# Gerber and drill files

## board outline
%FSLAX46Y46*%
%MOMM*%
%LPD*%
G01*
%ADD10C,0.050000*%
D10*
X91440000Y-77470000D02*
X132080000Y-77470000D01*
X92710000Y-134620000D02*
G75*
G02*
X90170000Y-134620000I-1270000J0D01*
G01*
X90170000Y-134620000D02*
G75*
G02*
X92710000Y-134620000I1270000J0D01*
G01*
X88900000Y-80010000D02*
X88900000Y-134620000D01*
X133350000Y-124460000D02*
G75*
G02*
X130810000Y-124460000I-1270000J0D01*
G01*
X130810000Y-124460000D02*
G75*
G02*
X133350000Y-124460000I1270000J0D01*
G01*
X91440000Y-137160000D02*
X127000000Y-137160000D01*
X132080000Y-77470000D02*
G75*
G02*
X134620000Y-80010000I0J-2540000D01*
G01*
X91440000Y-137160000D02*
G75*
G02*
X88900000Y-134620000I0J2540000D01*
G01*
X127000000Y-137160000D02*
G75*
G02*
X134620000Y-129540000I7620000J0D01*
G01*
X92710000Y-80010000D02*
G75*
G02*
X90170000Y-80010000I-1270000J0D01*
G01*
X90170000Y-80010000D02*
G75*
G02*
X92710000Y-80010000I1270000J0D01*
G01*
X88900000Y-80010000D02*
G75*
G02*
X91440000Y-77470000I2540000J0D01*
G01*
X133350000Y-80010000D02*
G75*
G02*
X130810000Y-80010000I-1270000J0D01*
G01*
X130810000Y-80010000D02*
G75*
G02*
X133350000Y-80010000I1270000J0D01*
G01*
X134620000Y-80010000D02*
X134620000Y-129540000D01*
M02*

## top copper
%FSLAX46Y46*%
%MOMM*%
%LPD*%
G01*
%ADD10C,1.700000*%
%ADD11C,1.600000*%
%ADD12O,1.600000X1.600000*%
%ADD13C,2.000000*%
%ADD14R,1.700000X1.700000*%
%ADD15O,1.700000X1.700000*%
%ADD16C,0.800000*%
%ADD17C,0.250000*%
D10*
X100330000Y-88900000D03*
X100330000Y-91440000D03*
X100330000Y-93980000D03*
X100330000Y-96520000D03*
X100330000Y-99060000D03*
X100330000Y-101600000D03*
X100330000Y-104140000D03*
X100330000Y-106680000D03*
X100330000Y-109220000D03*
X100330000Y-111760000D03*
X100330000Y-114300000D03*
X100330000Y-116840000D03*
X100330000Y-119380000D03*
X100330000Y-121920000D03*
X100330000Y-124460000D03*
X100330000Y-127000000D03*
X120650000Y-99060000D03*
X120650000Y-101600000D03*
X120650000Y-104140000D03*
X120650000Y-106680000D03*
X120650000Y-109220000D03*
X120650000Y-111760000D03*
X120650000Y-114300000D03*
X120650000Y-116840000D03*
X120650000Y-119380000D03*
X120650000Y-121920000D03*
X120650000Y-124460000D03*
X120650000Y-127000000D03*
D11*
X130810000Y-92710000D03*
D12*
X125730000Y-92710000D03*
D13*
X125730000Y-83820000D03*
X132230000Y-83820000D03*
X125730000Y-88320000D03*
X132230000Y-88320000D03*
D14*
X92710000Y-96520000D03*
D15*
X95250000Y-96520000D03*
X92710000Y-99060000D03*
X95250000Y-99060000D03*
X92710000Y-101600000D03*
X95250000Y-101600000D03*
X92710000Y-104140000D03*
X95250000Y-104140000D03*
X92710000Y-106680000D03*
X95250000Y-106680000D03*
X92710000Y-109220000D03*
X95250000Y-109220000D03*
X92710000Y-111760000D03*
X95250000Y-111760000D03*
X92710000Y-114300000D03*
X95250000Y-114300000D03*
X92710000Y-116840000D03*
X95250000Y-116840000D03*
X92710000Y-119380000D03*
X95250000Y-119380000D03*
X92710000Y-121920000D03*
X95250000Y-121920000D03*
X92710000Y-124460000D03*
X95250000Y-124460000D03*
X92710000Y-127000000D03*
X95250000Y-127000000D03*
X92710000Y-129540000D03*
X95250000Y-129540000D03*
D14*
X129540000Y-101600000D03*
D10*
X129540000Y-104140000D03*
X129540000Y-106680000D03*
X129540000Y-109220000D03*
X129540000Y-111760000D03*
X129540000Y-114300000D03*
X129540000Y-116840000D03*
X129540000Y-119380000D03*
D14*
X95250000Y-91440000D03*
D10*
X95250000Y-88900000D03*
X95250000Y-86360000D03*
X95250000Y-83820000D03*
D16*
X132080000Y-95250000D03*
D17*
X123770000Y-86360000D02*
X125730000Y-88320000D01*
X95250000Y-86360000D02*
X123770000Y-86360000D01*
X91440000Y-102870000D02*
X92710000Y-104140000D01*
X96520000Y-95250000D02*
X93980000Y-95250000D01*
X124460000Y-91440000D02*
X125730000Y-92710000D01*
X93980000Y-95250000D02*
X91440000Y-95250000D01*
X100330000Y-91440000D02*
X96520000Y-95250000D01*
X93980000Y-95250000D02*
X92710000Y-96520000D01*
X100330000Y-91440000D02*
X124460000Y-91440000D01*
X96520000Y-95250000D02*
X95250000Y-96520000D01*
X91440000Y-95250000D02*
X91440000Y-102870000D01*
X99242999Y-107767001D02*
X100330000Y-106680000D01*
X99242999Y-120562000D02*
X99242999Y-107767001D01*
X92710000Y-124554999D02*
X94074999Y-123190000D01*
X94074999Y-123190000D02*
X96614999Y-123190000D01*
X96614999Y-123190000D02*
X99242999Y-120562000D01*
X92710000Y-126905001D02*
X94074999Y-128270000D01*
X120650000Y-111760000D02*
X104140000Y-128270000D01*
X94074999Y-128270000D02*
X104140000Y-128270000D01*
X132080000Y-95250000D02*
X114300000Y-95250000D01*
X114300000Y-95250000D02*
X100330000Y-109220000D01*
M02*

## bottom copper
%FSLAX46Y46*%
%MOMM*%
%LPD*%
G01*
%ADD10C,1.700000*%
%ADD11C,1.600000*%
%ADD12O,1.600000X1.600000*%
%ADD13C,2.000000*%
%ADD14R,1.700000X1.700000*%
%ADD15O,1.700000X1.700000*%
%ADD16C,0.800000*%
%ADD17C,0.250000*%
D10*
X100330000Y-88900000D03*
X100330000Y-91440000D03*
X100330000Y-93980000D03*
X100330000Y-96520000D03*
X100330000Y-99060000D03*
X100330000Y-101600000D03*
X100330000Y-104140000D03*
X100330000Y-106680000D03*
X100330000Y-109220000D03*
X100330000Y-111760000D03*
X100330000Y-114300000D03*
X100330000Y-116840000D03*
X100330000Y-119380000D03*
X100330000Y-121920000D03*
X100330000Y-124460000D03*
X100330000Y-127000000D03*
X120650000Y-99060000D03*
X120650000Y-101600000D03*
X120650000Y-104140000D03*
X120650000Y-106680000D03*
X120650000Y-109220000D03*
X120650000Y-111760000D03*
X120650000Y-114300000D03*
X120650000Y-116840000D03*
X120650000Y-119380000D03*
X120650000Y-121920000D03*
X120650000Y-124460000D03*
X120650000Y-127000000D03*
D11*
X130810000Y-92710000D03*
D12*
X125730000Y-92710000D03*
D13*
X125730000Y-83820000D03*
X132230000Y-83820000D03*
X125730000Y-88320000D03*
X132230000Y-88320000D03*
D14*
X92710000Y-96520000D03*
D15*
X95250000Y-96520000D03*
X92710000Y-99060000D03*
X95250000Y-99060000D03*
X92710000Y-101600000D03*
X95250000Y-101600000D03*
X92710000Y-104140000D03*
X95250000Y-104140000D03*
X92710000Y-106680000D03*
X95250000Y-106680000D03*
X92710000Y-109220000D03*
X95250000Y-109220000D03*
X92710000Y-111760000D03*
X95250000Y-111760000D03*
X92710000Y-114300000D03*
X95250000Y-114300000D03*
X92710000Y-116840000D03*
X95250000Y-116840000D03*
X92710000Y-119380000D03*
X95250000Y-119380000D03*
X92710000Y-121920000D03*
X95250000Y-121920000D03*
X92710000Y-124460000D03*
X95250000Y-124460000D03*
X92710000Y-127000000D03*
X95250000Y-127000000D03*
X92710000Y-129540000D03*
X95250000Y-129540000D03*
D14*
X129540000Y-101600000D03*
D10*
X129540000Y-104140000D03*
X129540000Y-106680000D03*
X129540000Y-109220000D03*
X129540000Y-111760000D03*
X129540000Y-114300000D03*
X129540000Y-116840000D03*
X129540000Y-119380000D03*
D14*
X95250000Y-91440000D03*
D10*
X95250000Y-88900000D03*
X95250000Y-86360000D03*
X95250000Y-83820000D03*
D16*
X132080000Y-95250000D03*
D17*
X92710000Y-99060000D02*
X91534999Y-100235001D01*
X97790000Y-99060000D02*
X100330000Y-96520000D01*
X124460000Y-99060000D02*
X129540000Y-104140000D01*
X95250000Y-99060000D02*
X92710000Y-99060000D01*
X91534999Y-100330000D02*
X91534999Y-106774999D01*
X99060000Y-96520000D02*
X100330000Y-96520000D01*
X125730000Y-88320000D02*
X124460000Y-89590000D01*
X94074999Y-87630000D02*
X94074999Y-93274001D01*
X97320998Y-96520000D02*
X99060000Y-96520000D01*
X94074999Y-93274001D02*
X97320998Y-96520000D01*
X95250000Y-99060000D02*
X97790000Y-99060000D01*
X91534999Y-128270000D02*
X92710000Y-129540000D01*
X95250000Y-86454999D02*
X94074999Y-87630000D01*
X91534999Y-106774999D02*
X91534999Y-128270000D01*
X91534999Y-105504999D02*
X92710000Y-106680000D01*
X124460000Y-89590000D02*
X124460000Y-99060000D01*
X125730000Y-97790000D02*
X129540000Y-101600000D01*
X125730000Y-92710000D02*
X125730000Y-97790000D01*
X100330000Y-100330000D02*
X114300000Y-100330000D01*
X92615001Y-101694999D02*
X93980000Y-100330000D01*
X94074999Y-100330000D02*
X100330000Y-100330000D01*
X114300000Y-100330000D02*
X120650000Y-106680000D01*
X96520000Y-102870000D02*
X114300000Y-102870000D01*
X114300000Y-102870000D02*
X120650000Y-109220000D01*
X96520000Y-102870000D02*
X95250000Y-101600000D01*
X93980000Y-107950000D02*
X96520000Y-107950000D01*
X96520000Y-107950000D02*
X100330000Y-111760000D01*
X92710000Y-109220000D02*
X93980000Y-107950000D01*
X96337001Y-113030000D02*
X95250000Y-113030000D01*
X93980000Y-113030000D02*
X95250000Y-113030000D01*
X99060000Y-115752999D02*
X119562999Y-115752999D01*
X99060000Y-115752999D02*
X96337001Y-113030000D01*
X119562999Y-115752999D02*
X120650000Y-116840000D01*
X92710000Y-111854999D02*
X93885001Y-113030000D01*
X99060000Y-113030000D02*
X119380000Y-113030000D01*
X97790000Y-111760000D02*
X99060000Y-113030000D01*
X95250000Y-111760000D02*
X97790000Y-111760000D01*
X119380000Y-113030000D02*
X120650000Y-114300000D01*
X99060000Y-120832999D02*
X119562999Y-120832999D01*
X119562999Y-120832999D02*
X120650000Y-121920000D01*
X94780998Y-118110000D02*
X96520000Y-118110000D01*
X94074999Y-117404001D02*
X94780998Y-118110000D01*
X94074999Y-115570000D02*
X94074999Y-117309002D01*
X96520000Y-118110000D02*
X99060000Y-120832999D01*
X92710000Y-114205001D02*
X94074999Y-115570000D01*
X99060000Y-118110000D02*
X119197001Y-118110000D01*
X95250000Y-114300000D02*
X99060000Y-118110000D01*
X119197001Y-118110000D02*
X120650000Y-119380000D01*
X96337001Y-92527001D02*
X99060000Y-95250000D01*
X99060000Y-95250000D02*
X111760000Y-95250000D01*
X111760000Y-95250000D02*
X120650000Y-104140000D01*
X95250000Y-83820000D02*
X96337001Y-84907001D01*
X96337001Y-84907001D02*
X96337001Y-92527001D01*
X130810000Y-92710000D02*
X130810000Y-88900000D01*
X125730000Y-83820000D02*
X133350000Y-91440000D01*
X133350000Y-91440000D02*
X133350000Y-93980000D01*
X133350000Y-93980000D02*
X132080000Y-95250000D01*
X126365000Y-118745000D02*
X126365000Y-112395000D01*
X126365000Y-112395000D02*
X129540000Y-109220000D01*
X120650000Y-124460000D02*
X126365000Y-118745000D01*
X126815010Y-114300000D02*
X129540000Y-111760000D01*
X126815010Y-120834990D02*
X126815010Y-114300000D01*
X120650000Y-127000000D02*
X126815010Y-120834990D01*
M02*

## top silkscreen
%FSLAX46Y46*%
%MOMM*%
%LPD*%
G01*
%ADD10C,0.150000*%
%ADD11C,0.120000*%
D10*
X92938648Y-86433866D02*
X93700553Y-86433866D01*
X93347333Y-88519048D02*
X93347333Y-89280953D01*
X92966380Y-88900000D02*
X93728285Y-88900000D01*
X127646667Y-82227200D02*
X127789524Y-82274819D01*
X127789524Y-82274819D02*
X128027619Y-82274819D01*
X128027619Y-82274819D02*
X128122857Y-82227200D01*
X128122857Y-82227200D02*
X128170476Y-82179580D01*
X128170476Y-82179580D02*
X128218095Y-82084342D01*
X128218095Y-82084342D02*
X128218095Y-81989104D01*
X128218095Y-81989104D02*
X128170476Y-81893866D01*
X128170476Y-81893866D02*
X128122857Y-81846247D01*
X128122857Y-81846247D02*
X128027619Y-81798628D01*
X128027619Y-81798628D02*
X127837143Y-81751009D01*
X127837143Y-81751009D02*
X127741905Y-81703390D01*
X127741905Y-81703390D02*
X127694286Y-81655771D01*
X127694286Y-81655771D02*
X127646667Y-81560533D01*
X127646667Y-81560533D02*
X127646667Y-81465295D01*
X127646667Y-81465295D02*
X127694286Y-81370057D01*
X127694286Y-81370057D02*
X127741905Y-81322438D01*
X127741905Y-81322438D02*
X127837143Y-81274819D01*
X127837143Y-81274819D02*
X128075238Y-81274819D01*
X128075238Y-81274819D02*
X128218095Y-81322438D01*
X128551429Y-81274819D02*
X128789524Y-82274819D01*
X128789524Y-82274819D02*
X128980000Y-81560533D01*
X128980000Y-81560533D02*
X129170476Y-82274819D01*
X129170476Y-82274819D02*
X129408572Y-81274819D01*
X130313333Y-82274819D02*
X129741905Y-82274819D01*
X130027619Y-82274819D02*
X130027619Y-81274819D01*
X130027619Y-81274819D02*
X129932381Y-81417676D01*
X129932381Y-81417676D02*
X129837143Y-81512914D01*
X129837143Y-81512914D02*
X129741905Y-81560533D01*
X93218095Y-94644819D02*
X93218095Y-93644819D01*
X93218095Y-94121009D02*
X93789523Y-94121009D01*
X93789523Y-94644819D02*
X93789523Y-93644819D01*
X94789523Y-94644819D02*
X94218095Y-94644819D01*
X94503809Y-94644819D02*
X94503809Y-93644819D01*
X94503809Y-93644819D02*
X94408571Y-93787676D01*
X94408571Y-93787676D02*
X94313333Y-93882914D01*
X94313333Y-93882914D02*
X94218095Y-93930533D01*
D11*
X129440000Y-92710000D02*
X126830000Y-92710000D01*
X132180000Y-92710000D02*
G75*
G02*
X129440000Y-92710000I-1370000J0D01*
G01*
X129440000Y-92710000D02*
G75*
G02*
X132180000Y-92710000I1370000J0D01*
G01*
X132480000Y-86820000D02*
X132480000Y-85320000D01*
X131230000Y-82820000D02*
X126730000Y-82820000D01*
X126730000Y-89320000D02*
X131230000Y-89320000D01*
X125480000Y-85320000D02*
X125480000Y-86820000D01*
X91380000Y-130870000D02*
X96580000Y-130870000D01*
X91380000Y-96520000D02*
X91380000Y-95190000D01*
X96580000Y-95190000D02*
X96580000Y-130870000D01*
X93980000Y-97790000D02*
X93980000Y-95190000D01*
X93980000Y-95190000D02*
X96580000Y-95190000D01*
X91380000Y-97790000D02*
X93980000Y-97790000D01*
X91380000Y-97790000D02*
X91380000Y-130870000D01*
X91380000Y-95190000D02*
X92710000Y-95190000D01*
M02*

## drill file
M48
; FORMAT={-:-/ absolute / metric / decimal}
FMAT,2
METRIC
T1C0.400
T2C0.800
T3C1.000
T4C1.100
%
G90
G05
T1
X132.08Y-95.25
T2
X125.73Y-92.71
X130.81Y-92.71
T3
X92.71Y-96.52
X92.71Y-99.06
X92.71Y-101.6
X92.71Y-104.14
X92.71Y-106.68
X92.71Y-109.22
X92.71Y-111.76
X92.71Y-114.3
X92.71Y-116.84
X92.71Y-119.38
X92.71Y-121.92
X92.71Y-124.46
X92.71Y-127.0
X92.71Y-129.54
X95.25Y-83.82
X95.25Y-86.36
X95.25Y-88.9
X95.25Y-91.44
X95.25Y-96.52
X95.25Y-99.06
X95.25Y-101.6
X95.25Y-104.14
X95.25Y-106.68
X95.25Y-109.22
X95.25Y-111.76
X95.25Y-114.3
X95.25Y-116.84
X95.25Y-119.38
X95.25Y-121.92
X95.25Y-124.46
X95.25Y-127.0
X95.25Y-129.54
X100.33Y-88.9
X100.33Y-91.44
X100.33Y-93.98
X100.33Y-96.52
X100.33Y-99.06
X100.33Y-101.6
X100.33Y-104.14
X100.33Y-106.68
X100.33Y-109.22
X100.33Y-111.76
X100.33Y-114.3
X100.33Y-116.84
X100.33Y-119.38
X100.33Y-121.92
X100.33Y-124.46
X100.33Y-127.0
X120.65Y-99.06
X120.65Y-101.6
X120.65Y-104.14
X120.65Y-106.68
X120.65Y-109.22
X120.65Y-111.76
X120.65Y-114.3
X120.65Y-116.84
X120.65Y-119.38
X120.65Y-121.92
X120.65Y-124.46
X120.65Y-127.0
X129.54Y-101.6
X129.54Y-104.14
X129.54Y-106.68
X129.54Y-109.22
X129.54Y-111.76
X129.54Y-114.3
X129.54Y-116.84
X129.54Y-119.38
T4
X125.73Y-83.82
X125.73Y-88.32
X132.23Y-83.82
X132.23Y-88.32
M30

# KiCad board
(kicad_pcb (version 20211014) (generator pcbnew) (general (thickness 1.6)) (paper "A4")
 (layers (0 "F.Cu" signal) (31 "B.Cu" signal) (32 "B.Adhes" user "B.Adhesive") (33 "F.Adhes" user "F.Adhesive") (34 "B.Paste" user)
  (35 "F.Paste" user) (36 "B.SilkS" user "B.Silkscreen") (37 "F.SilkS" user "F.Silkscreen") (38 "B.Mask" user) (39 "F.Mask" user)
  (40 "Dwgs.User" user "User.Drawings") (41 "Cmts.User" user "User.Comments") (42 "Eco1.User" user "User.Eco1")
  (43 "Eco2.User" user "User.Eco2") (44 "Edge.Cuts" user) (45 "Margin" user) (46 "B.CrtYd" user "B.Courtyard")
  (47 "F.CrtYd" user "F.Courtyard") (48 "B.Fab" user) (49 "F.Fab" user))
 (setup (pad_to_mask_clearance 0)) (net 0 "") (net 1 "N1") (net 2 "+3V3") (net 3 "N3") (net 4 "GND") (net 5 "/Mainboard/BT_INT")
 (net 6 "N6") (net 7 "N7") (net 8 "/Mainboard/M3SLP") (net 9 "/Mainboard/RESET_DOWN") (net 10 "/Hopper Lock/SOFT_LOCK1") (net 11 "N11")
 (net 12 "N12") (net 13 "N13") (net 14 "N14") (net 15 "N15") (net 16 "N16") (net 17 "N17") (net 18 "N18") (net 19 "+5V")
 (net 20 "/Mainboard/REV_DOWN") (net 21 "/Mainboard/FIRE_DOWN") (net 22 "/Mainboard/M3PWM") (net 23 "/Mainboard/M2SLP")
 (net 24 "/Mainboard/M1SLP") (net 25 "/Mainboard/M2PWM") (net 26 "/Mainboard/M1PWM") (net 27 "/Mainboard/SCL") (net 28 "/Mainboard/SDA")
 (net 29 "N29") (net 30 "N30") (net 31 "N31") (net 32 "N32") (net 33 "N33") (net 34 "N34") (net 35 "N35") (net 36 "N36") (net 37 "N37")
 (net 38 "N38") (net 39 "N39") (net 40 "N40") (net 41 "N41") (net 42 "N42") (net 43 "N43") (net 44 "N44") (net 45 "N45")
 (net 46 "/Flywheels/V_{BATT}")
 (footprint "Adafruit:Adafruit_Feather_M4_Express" (layer "F.Cu") (at 110.49 107.95)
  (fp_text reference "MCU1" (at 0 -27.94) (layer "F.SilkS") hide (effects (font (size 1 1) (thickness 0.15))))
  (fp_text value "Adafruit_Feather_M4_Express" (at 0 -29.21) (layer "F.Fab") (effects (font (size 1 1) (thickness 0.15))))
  (pad "1" thru_hole circle (at -10.16 -19.05) (size 1.7 1.7) (drill 1) (layers *.Cu *.Mask) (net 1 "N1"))
  (pad "2" thru_hole circle (at -10.16 -16.51) (size 1.7 1.7) (drill 1) (layers *.Cu *.Mask) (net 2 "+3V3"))
  (pad "3" thru_hole circle (at -10.16 -13.97) (size 1.7 1.7) (drill 1) (layers *.Cu *.Mask) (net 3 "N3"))
  (pad "4" thru_hole circle (at -10.16 -11.43) (size 1.7 1.7) (drill 1) (layers *.Cu *.Mask) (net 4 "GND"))
  (pad "5" thru_hole circle (at -10.16 -8.89) (size 1.7 1.7) (drill 1) (layers *.Cu *.Mask) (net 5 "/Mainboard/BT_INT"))
  (pad "6" thru_hole circle (at -10.16 -6.35) (size 1.7 1.7) (drill 1) (layers *.Cu *.Mask) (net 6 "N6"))
  (pad "7" thru_hole circle (at -10.16 -3.81) (size 1.7 1.7) (drill 1) (layers *.Cu *.Mask) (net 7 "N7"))
  (pad "8" thru_hole circle (at -10.16 -1.27) (size 1.7 1.7) (drill 1) (layers *.Cu *.Mask) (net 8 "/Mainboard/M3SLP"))
  (pad "9" thru_hole circle (at -10.16 1.27) (size 1.7 1.7) (drill 1) (layers *.Cu *.Mask) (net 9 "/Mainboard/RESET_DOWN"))
  (pad "10" thru_hole circle (at -10.16 3.81) (size 1.7 1.7) (drill 1) (layers *.Cu *.Mask) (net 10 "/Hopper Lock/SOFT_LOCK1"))
  (pad "11" thru_hole circle (at -10.16 6.35) (size 1.7 1.7) (drill 1) (layers *.Cu *.Mask) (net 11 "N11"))
  (pad "12" thru_hole circle (at -10.16 8.89) (size 1.7 1.7) (drill 1) (layers *.Cu *.Mask) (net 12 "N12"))
  (pad "13" thru_hole circle (at -10.16 11.43) (size 1.7 1.7) (drill 1) (layers *.Cu *.Mask) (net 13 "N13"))
  (pad "14" thru_hole circle (at -10.16 13.97) (size 1.7 1.7) (drill 1) (layers *.Cu *.Mask) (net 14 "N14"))
  (pad "15" thru_hole circle (at -10.16 16.51) (size 1.7 1.7) (drill 1) (layers *.Cu *.Mask) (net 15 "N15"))
  (pad "16" thru_hole circle (at -10.16 19.05) (size 1.7 1.7) (drill 1) (layers *.Cu *.Mask) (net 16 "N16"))
  (pad "17" thru_hole circle (at 10.16 -8.89) (size 1.7 1.7) (drill 1) (layers *.Cu *.Mask) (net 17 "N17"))
  (pad "18" thru_hole circle (at 10.16 -6.35) (size 1.7 1.7) (drill 1) (layers *.Cu *.Mask) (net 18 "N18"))
  (pad "19" thru_hole circle (at 10.16 -3.81) (size 1.7 1.7) (drill 1) (layers *.Cu *.Mask) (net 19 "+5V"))
  (pad "20" thru_hole circle (at 10.16 -1.27) (size 1.7 1.7) (drill 1) (layers *.Cu *.Mask) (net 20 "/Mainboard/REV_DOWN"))
  (pad "21" thru_hole circle (at 10.16 1.27) (size 1.7 1.7) (drill 1) (layers *.Cu *.Mask) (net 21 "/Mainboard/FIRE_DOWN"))
  (pad "22" thru_hole circle (at 10.16 3.81) (size 1.7 1.7) (drill 1) (layers *.Cu *.Mask) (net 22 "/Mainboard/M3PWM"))
  (pad "23" thru_hole circle (at 10.16 6.35) (size 1.7 1.7) (drill 1) (layers *.Cu *.Mask) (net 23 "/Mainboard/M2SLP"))
  (pad "24" thru_hole circle (at 10.16 8.89) (size 1.7 1.7) (drill 1) (layers *.Cu *.Mask) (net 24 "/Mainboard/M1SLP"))
  (pad "25" thru_hole circle (at 10.16 11.43) (size 1.7 1.7) (drill 1) (layers *.Cu *.Mask) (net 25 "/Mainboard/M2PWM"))
  (pad "26" thru_hole circle (at 10.16 13.97) (size 1.7 1.7) (drill 1) (layers *.Cu *.Mask) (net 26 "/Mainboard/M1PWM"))
  (pad "27" thru_hole circle (at 10.16 16.51) (size 1.7 1.7) (drill 1) (layers *.Cu *.Mask) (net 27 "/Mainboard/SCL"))
  (pad "28" thru_hole circle (at 10.16 19.05) (size 1.7 1.7) (drill 1) (layers *.Cu *.Mask) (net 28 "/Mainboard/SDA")))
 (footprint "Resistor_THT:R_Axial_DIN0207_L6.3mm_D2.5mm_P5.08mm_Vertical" (layer "F.Cu") (at 130.81 92.71 180)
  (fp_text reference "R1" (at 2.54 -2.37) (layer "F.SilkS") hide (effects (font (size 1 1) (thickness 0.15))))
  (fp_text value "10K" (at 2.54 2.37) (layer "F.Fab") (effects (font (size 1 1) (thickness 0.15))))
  (fp_line (start 1.37 0) (end 3.98 0) (layer "F.SilkS") (width 0.12))
  (fp_circle (center 0 0) (end 1.37 0) (layer "F.SilkS") (width 0.12) (fill none))
  (pad "1" thru_hole circle locked (at 0 0 180) (size 1.6 1.6) (drill 0.8) (layers *.Cu *.Mask) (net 9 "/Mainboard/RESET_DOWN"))
  (pad "2" thru_hole oval locked (at 5.08 0 180) (size 1.6 1.6) (drill 0.8) (layers *.Cu *.Mask) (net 2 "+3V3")))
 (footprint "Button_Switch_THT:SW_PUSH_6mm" (layer "F.Cu") (at 125.73 83.82)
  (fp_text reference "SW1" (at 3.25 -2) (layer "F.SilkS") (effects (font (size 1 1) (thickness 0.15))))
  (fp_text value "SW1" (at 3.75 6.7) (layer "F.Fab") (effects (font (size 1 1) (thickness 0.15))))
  (fp_line (start 6.75 3) (end 6.75 1.5) (layer "F.SilkS") (width 0.12))
  (fp_line (start 5.5 -1) (end 1 -1) (layer "F.SilkS") (width 0.12))
  (fp_line (start 1 5.5) (end 5.5 5.5) (layer "F.SilkS") (width 0.12))
  (fp_line (start -0.25 1.5) (end -0.25 3) (layer "F.SilkS") (width 0.12))
  (pad "1" thru_hole circle locked (at 0 0 90) (size 2 2) (drill 1.1) (layers *.Cu *.Mask) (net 9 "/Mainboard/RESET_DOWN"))
  (pad "1" thru_hole circle locked (at 6.5 0 90) (size 2 2) (drill 1.1) (layers *.Cu *.Mask) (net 9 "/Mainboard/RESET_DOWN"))
  (pad "2" thru_hole circle locked (at 0 4.5 90) (size 2 2) (drill 1.1) (layers *.Cu *.Mask) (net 4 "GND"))
  (pad "2" thru_hole circle locked (at 6.5 4.5 90) (size 2 2) (drill 1.1) (layers *.Cu *.Mask) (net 4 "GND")))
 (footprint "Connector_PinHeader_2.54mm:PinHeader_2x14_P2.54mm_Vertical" (layer "F.Cu") (at 92.71 96.52)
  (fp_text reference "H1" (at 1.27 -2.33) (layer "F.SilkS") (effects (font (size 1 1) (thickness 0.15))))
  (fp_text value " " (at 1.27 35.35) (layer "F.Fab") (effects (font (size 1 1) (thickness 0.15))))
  (fp_line (start -1.33 34.35) (end 3.87 34.35) (layer "F.SilkS") (width 0.12))
  (fp_line (start -1.33 0) (end -1.33 -1.33) (layer "F.SilkS") (width 0.12))
  (fp_line (start 3.87 -1.33) (end 3.87 34.35) (layer "F.SilkS") (width 0.12))
  (fp_line (start 1.27 1.27) (end 1.27 -1.33) (layer "F.SilkS") (width 0.12))
  (fp_line (start 1.27 -1.33) (end 3.87 -1.33) (layer "F.SilkS") (width 0.12))
  (fp_line (start -1.33 1.27) (end 1.27 1.27) (layer "F.SilkS") (width 0.12))
  (fp_line (start -1.33 1.27) (end -1.33 34.35) (layer "F.SilkS") (width 0.12))
  (fp_line (start -1.33 -1.33) (end 0 -1.33) (layer "F.SilkS") (width 0.12))
  (pad "1" thru_hole rect locked (at 0 0) (size 1.7 1.7) (drill 1) (layers *.Cu *.Mask) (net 2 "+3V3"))
  (pad "2" thru_hole oval locked (at 2.54 0) (size 1.7 1.7) (drill 1) (layers *.Cu *.Mask) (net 2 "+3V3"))
  (pad "3" thru_hole oval locked (at 0 2.54) (size 1.7 1.7) (drill 1) (layers *.Cu *.Mask) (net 4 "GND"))
  (pad "4" thru_hole oval locked (at 2.54 2.54) (size 1.7 1.7) (drill 1) (layers *.Cu *.Mask) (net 4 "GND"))
  (pad "5" thru_hole oval locked (at 0 5.08) (size 1.7 1.7) (drill 1) (layers *.Cu *.Mask) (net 20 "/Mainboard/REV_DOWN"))
  (pad "6" thru_hole oval locked (at 2.54 5.08) (size 1.7 1.7) (drill 1) (layers *.Cu *.Mask) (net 21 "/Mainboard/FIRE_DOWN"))
  (pad "7" thru_hole oval locked (at 0 7.62) (size 1.7 1.7) (drill 1) (layers *.Cu *.Mask) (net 2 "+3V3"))
  (pad "8" thru_hole oval locked (at 2.54 7.62) (size 1.7 1.7) (drill 1) (layers *.Cu *.Mask) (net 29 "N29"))
  (pad "9" thru_hole oval locked (at 0 10.16) (size 1.7 1.7) (drill 1) (layers *.Cu *.Mask) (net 4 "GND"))
  (pad "10" thru_hole oval locked (at 2.54 10.16) (size 1.7 1.7) (drill 1) (layers *.Cu *.Mask) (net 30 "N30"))
  (pad "11" thru_hole oval locked (at 0 12.7) (size 1.7 1.7) (drill 1) (layers *.Cu *.Mask) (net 10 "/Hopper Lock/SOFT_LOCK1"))
  (pad "12" thru_hole oval locked (at 2.54 12.7) (size 1.7 1.7) (drill 1) (layers *.Cu *.Mask) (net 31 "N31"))
  (pad "13" thru_hole oval locked (at 0 15.24) (size 1.7 1.7) (drill 1) (layers *.Cu *.Mask) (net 24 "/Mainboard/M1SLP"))
  (pad "14" thru_hole oval locked (at 2.54 15.24) (size 1.7 1.7) (drill 1) (layers *.Cu *.Mask) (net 23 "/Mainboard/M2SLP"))
  (pad "15" thru_hole oval locked (at 0 17.78) (size 1.7 1.7) (drill 1) (layers *.Cu *.Mask) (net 26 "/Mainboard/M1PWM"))
  (pad "16" thru_hole oval locked (at 2.54 17.78) (size 1.7 1.7) (drill 1) (layers *.Cu *.Mask) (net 25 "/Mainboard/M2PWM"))
  (pad "17" thru_hole oval locked (at 0 20.32) (size 1.7 1.7) (drill 1) (layers *.Cu *.Mask) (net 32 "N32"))
  (pad "18" thru_hole oval locked (at 2.54 20.32) (size 1.7 1.7) (drill 1) (layers *.Cu *.Mask) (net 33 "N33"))
  (pad "19" thru_hole oval locked (at 0 22.86) (size 1.7 1.7) (drill 1) (layers *.Cu *.Mask) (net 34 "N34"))
  (pad "20" thru_hole oval locked (at 2.54 22.86) (size 1.7 1.7) (drill 1) (layers *.Cu *.Mask) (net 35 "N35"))
  (pad "21" thru_hole oval locked (at 0 25.4) (size 1.7 1.7) (drill 1) (layers *.Cu *.Mask) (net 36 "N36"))
  (pad "22" thru_hole oval locked (at 2.54 25.4) (size 1.7 1.7) (drill 1) (layers *.Cu *.Mask) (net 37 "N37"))
  (pad "23" thru_hole oval locked (at 0 27.94) (size 1.7 1.7) (drill 1) (layers *.Cu *.Mask) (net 8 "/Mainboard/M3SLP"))
  (pad "24" thru_hole oval locked (at 2.54 27.94) (size 1.7 1.7) (drill 1) (layers *.Cu *.Mask) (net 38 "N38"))
  (pad "25" thru_hole oval locked (at 0 30.48) (size 1.7 1.7) (drill 1) (layers *.Cu *.Mask) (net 22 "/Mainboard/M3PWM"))
  (pad "26" thru_hole oval locked (at 2.54 30.48) (size 1.7 1.7) (drill 1) (layers *.Cu *.Mask) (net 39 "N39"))
  (pad "27" thru_hole oval locked (at 0 33.02) (size 1.7 1.7) (drill 1) (layers *.Cu *.Mask) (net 4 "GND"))
  (pad "28" thru_hole oval locked (at 2.54 33.02) (size 1.7 1.7) (drill 1) (layers *.Cu *.Mask) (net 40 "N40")))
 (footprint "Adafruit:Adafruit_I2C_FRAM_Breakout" (layer "B.Cu") (at 124.46 110.49 -90)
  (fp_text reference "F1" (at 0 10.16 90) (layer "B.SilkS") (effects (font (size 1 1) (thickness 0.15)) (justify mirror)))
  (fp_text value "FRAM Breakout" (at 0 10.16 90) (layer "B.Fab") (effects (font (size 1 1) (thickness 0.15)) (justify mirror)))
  (pad "1" thru_hole rect (at -8.89 -5.08 270) (size 1.7 1.7) (drill 1) (layers *.Cu *.Mask) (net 2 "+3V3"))
  (pad "2" thru_hole circle (at -6.35 -5.08 270) (size 1.7 1.7) (drill 1) (layers *.Cu *.Mask) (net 4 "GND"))
  (pad "3" thru_hole circle (at -3.81 -5.08 270) (size 1.7 1.7) (drill 1) (layers *.Cu *.Mask) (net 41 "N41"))
  (pad "4" thru_hole circle (at -1.27 -5.08 270) (size 1.7 1.7) (drill 1) (layers *.Cu *.Mask) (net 27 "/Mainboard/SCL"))
  (pad "5" thru_hole circle (at 1.27 -5.08 270) (size 1.7 1.7) (drill 1) (layers *.Cu *.Mask) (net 28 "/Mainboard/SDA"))
  (pad "6" thru_hole circle (at 3.81 -5.08 270) (size 1.7 1.7) (drill 1) (layers *.Cu *.Mask) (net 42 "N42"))
  (pad "7" thru_hole circle (at 6.35 -5.08 270) (size 1.7 1.7) (drill 1) (layers *.Cu *.Mask) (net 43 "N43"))
  (pad "8" thru_hole circle (at 8.89 -5.08 270) (size 1.7 1.7) (drill 1) (layers *.Cu *.Mask) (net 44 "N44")))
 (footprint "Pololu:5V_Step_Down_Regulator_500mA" (layer "B.Cu") (at 100.33 87.63 90)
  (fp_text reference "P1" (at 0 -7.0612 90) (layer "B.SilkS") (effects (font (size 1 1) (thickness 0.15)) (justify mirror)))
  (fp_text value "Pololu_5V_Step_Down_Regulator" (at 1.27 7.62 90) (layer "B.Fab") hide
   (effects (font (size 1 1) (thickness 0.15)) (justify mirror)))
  (pad "1" thru_hole rect (at -3.81 -5.08 90) (size 1.7 1.7) (drill 1) (layers *.Cu *.Mask) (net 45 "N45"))
  (pad "2" thru_hole circle (at -1.27 -5.08 90) (size 1.7 1.7) (drill 1) (layers *.Cu *.Mask) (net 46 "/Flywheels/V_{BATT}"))
  (pad "3" thru_hole circle (at 1.27 -5.08 90) (size 1.7 1.7) (drill 1) (layers *.Cu *.Mask) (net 4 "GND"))
  (pad "4" thru_hole circle (at 3.81 -5.08 90) (size 1.7 1.7) (drill 1) (layers *.Cu *.Mask) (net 19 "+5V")))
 (gr_line (start 91.44 77.47) (end 132.08 77.47) (layer "Edge.Cuts") (width 0.05))
 (gr_circle (center 91.44 134.62) (end 91.44 135.89) (layer "Edge.Cuts") (width 0.05) (fill none))
 (gr_line (start 88.9 80.01) (end 88.9 134.62) (layer "Edge.Cuts") (width 0.05))
 (gr_circle (center 132.08 124.46) (end 133.35 124.46) (layer "Edge.Cuts") (width 0.05) (fill none))
 (gr_line (start 91.44 137.16) (end 127 137.16) (layer "Edge.Cuts") (width 0.05))
 (gr_arc (start 132.08 77.47) (mid 133.876051 78.213949) (end 134.62 80.01) (layer "Edge.Cuts") (width 0.05))
 (gr_arc (start 91.44 137.16) (mid 89.643949 136.416051) (end 88.9 134.62) (layer "Edge.Cuts") (width 0.05))
 (gr_arc (start 127 137.16) (mid 129.231846 131.771846) (end 134.62 129.54) (layer "Edge.Cuts") (width 0.05))
 (gr_circle (center 91.44 80.01) (end 90.17 80.01) (layer "Edge.Cuts") (width 0.05) (fill none))
 (gr_arc (start 88.9 80.01) (mid 89.643949 78.213949) (end 91.44 77.47) (layer "Edge.Cuts") (width 0.05))
 (gr_circle (center 132.08 80.01) (end 133.35 80.01) (layer "Edge.Cuts") (width 0.05) (fill none))
 (gr_line (start 134.62 80.01) (end 134.62 129.54) (layer "Edge.Cuts") (width 0.05))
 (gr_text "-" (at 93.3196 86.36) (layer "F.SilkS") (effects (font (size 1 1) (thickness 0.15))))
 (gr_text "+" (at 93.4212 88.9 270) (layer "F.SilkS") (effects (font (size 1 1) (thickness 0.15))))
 (segment (start 123.77 86.36) (end 125.73 88.32) (width 0.25) (layer "F.Cu") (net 4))
 (segment (start 95.25 86.36) (end 123.77 86.36) (width 0.25) (layer "F.Cu") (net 4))
 (segment (start 92.71 99.06) (end 91.534999 100.235001) (width 0.25) (layer "B.Cu") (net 4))
 (segment (start 97.79 99.06) (end 100.33 96.52) (width 0.25) (layer "B.Cu") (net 4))
 (segment (start 124.46 99.06) (end 129.54 104.14) (width 0.25) (layer "B.Cu") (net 4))
 (segment (start 95.25 99.06) (end 92.71 99.06) (width 0.25) (layer "B.Cu") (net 4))
 (segment (start 91.534999 100.33) (end 91.534999 106.774999) (width 0.25) (layer "B.Cu") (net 4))
 (segment (start 99.06 96.52) (end 100.33 96.52) (width 0.25) (layer "B.Cu") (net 4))
 (segment (start 125.73 88.32) (end 124.46 89.59) (width 0.25) (layer "B.Cu") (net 4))
 (segment (start 94.074999 87.63) (end 94.074999 93.274001) (width 0.25) (layer "B.Cu") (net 4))
 (segment (start 97.320998 96.52) (end 99.06 96.52) (width 0.25) (layer "B.Cu") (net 4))
 (segment (start 94.074999 93.274001) (end 97.320998 96.52) (width 0.25) (layer "B.Cu") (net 4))
 (segment (start 95.25 99.06) (end 97.79 99.06) (width 0.25) (layer "B.Cu") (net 4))
 (segment (start 91.534999 128.27) (end 92.71 129.54) (width 0.25) (layer "B.Cu") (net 4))
 (segment (start 95.25 86.454999) (end 94.074999 87.63) (width 0.25) (layer "B.Cu") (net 4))
 (segment (start 91.534999 106.774999) (end 91.534999 128.27) (width 0.25) (layer "B.Cu") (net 4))
 (segment (start 91.534999 105.504999) (end 92.71 106.68) (width 0.25) (layer "B.Cu") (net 4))
 (segment (start 124.46 89.59) (end 124.46 99.06) (width 0.25) (layer "B.Cu") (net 4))
 (segment (start 91.44 102.87) (end 92.71 104.14) (width 0.25) (layer "F.Cu") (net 2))
 (segment (start 96.52 95.25) (end 93.98 95.25) (width 0.25) (layer "F.Cu") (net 2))
 (segment (start 124.46 91.44) (end 125.73 92.71) (width 0.25) (layer "F.Cu") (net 2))
 (segment (start 93.98 95.25) (end 91.44 95.25) (width 0.25) (layer "F.Cu") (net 2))
 (segment (start 100.33 91.44) (end 96.52 95.25) (width 0.25) (layer "F.Cu") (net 2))
 (segment (start 93.98 95.25) (end 92.71 96.52) (width 0.25) (layer "F.Cu") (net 2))
 (segment (start 100.33 91.44) (end 124.46 91.44) (width 0.25) (layer "F.Cu") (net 2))
 (segment (start 96.52 95.25) (end 95.25 96.52) (width 0.25) (layer "F.Cu") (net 2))
 (segment (start 91.44 95.25) (end 91.44 102.87) (width 0.25) (layer "F.Cu") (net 2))
 (segment (start 125.73 97.79) (end 129.54 101.6) (width 0.25) (layer "B.Cu") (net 2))
 (segment (start 125.73 92.71) (end 125.73 97.79) (width 0.25) (layer "B.Cu") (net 2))
 (segment (start 100.33 100.33) (end 114.3 100.33) (width 0.25) (layer "B.Cu") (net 20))
 (segment (start 92.615001 101.694999) (end 93.98 100.33) (width 0.25) (layer "B.Cu") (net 20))
 (segment (start 94.074999 100.33) (end 100.33 100.33) (width 0.25) (layer "B.Cu") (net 20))
 (segment (start 114.3 100.33) (end 120.65 106.68) (width 0.25) (layer "B.Cu") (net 20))
 (segment (start 96.52 102.87) (end 114.3 102.87) (width 0.25) (layer "B.Cu") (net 21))
 (segment (start 114.3 102.87) (end 120.65 109.22) (width 0.25) (layer "B.Cu") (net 21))
 (segment (start 96.52 102.87) (end 95.25 101.6) (width 0.25) (layer "B.Cu") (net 21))
 (segment (start 93.98 107.95) (end 96.52 107.95) (width 0.25) (layer "B.Cu") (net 10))
 (segment (start 96.52 107.95) (end 100.33 111.76) (width 0.25) (layer "B.Cu") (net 10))
 (segment (start 92.71 109.22) (end 93.98 107.95) (width 0.25) (layer "B.Cu") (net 10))
 (segment (start 96.337001 113.03) (end 95.25 113.03) (width 0.25) (layer "B.Cu") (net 24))
 (segment (start 93.98 113.03) (end 95.25 113.03) (width 0.25) (layer "B.Cu") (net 24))
 (segment (start 99.06 115.752999) (end 119.562999 115.752999) (width 0.25) (layer "B.Cu") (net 24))
 (segment (start 99.06 115.752999) (end 96.337001 113.03) (width 0.25) (layer "B.Cu") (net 24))
 (segment (start 119.562999 115.752999) (end 120.65 116.84) (width 0.25) (layer "B.Cu") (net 24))
 (segment (start 92.71 111.854999) (end 93.885001 113.03) (width 0.25) (layer "B.Cu") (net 24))
 (segment (start 99.06 113.03) (end 119.38 113.03) (width 0.25) (layer "B.Cu") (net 23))
 (segment (start 97.79 111.76) (end 99.06 113.03) (width 0.25) (layer "B.Cu") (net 23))
 (segment (start 95.25 111.76) (end 97.79 111.76) (width 0.25) (layer "B.Cu") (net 23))
 (segment (start 119.38 113.03) (end 120.65 114.3) (width 0.25) (layer "B.Cu") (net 23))
 (segment (start 99.06 120.832999) (end 119.562999 120.832999) (width 0.25) (layer "B.Cu") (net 26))
 (segment (start 119.562999 120.832999) (end 120.65 121.92) (width 0.25) (layer "B.Cu") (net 26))
 (segment (start 94.780998 118.11) (end 96.52 118.11) (width 0.25) (layer "B.Cu") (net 26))
 (segment (start 94.074999 117.404001) (end 94.780998 118.11) (width 0.25) (layer "B.Cu") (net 26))
 (segment (start 94.074999 115.57) (end 94.074999 117.309002) (width 0.25) (layer "B.Cu") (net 26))
 (segment (start 96.52 118.11) (end 99.06 120.832999) (width 0.25) (layer "B.Cu") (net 26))
 (segment (start 92.71 114.205001) (end 94.074999 115.57) (width 0.25) (layer "B.Cu") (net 26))
 (segment (start 99.06 118.11) (end 119.197001 118.11) (width 0.25) (layer "B.Cu") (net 25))
 (segment (start 95.25 114.3) (end 99.06 118.11) (width 0.25) (layer "B.Cu") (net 25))
 (segment (start 119.197001 118.11) (end 120.65 119.38) (width 0.25) (layer "B.Cu") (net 25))
 (segment (start 99.242999 107.767001) (end 100.33 106.68) (width 0.25) (layer "F.Cu") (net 8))
 (segment (start 99.242999 120.562) (end 99.242999 107.767001) (width 0.25) (layer "F.Cu") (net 8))
 (segment (start 92.71 124.554999) (end 94.074999 123.19) (width 0.25) (layer "F.Cu") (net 8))
 (segment (start 94.074999 123.19) (end 96.614999 123.19) (width 0.25) (layer "F.Cu") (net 8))
 (segment (start 96.614999 123.19) (end 99.242999 120.562) (width 0.25) (layer "F.Cu") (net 8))
 (segment (start 92.71 126.905001) (end 94.074999 128.27) (width 0.25) (layer "F.Cu") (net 22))
 (segment (start 120.65 111.76) (end 104.14 128.27) (width 0.25) (layer "F.Cu") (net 22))
 (segment (start 94.074999 128.27) (end 104.14 128.27) (width 0.25) (layer "F.Cu") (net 22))
 (segment (start 96.337001 92.527001) (end 99.06 95.25) (width 0.25) (layer "B.Cu") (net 19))
 (segment (start 99.06 95.25) (end 111.76 95.25) (width 0.25) (layer "B.Cu") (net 19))
 (segment (start 111.76 95.25) (end 120.65 104.14) (width 0.25) (layer "B.Cu") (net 19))
 (segment (start 95.25 83.82) (end 96.337001 84.907001) (width 0.25) (layer "B.Cu") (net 19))
 (segment (start 96.337001 84.907001) (end 96.337001 92.527001) (width 0.25) (layer "B.Cu") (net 19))
 (segment (start 132.08 95.25) (end 114.3 95.25) (width 0.25) (layer "F.Cu") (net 9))
 (segment (start 114.3 95.25) (end 100.33 109.22) (width 0.25) (layer "F.Cu") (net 9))
 (via (at 132.08 95.25) (size 0.8) (drill 0.4) (layers "F.Cu" "B.Cu") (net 9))
 (segment (start 130.81 92.71) (end 130.81 88.9) (width 0.25) (layer "B.Cu") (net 9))
 (segment (start 125.73 83.82) (end 133.35 91.44) (width 0.25) (layer "B.Cu") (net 9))
 (segment (start 133.35 91.44) (end 133.35 93.98) (width 0.25) (layer "B.Cu") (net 9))
 (segment (start 133.35 93.98) (end 132.08 95.25) (width 0.25) (layer "B.Cu") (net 9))
 (segment (start 126.365 118.745) (end 126.365 112.395) (width 0.25) (layer "B.Cu") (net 27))
 (segment (start 126.365 112.395) (end 129.54 109.22) (width 0.25) (layer "B.Cu") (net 27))
 (segment (start 120.65 124.46) (end 126.365 118.745) (width 0.25) (layer "B.Cu") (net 27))
 (segment (start 126.81501 114.3) (end 129.54 111.76) (width 0.25) (layer "B.Cu") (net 28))
 (segment (start 126.81501 120.83499) (end 126.81501 114.3) (width 0.25) (layer "B.Cu") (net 28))
 (segment (start 120.65 127) (end 126.81501 120.83499) (width 0.25) (layer "B.Cu") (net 28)))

